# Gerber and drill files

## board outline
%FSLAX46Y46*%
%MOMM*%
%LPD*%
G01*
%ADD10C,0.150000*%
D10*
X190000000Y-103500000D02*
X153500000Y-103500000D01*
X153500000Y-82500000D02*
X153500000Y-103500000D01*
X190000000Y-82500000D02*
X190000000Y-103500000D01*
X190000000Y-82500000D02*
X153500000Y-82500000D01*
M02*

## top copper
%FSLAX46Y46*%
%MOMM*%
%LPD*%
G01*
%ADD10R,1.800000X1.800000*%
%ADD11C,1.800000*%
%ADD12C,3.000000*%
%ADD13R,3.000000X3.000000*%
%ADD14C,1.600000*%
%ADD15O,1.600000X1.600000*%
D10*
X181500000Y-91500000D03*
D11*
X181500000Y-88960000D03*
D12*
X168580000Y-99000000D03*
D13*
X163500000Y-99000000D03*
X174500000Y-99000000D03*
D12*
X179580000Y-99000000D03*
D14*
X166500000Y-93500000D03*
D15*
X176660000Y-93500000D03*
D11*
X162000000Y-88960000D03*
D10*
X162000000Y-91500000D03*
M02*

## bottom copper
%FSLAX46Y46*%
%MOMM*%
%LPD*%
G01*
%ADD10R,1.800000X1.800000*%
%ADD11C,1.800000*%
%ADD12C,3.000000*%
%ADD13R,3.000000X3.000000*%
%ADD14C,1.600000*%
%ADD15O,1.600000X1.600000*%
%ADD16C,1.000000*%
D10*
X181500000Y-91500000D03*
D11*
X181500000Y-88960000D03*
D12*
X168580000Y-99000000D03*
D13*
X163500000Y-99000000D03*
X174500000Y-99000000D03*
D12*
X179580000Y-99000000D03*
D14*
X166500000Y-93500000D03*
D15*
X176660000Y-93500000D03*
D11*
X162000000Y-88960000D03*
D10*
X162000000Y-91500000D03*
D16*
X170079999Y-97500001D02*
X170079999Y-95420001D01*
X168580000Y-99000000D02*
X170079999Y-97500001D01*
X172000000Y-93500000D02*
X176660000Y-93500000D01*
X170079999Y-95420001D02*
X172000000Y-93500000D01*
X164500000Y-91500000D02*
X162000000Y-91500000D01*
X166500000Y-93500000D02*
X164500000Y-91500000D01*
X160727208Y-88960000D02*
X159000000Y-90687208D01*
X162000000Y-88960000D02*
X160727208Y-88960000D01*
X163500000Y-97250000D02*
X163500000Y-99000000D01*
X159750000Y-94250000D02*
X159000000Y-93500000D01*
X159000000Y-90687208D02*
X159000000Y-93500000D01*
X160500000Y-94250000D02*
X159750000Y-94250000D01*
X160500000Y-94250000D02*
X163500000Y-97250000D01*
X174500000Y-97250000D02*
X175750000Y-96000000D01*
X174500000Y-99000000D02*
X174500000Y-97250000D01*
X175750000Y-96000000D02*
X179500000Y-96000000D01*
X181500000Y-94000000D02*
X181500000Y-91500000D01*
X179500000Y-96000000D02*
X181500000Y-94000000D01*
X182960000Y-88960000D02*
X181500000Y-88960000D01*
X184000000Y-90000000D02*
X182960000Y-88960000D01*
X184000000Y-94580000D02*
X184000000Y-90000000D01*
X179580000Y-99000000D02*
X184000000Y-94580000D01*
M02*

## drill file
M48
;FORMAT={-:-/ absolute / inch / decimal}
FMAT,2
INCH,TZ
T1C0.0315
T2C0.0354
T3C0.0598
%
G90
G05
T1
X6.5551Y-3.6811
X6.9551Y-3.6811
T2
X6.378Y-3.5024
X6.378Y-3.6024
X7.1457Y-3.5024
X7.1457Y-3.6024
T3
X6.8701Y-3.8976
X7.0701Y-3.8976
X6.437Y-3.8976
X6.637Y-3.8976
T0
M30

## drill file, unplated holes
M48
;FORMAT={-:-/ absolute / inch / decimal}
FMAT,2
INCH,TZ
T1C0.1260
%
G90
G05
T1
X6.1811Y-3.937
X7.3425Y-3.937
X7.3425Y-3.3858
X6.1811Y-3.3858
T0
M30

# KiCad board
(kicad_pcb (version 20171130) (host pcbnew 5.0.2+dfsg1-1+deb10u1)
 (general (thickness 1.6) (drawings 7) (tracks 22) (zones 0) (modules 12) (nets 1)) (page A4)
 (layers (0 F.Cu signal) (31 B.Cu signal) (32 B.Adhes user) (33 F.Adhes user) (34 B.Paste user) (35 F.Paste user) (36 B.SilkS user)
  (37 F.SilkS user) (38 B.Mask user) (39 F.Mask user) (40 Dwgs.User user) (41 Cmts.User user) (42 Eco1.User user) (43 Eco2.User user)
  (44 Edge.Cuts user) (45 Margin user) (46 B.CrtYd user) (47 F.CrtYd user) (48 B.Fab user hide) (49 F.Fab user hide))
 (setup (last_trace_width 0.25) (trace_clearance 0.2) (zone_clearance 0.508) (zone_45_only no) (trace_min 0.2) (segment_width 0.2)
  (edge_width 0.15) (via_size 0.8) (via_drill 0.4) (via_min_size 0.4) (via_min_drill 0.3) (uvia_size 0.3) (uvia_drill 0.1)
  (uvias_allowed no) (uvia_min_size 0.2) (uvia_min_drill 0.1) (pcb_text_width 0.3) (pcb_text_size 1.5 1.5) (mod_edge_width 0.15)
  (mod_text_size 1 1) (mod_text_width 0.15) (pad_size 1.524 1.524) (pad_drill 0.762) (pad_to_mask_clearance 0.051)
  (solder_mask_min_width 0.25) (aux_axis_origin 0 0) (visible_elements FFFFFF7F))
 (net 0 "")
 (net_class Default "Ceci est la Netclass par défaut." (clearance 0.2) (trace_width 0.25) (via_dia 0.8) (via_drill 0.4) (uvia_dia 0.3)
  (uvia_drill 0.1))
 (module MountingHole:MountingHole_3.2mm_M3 (layer F.Cu) (at 157 100)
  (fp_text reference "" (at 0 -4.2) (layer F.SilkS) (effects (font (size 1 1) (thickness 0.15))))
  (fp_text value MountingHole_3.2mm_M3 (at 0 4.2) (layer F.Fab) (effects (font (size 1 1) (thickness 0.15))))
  (pad 1 np_thru_hole circle (at 0 0) (size 3.2 3.2) (drill 3.2) (layers *.Cu *.Mask)))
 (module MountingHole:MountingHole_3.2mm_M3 (layer F.Cu) (at 186.5 100)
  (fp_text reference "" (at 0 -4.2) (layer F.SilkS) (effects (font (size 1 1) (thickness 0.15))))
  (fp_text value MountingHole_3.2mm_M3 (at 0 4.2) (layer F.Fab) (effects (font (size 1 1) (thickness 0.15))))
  (pad 1 np_thru_hole circle (at 0 0) (size 3.2 3.2) (drill 3.2) (layers *.Cu *.Mask)))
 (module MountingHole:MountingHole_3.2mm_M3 (layer F.Cu) (at 186.5 86)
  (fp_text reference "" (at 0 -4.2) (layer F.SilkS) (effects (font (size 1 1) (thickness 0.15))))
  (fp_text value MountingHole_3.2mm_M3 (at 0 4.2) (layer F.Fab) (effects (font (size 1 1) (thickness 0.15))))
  (pad 1 np_thru_hole circle (at 0 0) (size 3.2 3.2) (drill 3.2) (layers *.Cu *.Mask)))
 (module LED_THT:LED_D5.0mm (layer F.Cu) (at 181.5 91.5 90)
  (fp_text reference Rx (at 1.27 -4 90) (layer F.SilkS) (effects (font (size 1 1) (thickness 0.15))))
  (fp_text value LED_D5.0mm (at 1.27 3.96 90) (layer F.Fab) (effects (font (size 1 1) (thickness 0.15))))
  (pad 1 thru_hole rect (at 0 0 90) (size 1.8 1.8) (drill 0.9) (layers *.Cu *.Mask))
  (pad 2 thru_hole circle (at 2.54 0 90) (size 1.8 1.8) (drill 0.9) (layers *.Cu *.Mask)))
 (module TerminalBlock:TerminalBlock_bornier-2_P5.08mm (layer F.Cu) (at 163.5 99)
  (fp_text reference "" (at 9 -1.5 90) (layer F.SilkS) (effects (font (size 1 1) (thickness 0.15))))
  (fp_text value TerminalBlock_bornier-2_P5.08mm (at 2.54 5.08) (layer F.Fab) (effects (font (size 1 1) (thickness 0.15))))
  (pad 2 thru_hole circle (at 5.08 0) (size 3 3) (drill 1.52) (layers *.Cu *.Mask))
  (pad 1 thru_hole rect (at 0 0) (size 3 3) (drill 1.52) (layers *.Cu *.Mask)))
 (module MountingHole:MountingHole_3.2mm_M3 (layer F.Cu) (at 157 86)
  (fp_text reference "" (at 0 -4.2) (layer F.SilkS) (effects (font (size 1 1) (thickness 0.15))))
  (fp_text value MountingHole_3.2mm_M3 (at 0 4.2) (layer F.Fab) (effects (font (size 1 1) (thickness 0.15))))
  (pad 1 np_thru_hole circle (at 0 0) (size 3.2 3.2) (drill 3.2) (layers *.Cu *.Mask)))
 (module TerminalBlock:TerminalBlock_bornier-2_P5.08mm (layer F.Cu) (at 174.5 99)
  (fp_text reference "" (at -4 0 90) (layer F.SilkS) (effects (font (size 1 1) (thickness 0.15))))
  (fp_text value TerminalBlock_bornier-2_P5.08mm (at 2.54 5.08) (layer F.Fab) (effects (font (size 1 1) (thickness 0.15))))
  (pad 1 thru_hole rect (at 0 0) (size 3 3) (drill 1.52) (layers *.Cu *.Mask))
  (pad 2 thru_hole circle (at 5.08 0) (size 3 3) (drill 1.52) (layers *.Cu *.Mask)))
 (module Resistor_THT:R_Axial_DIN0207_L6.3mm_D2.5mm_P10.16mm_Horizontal (layer F.Cu) (at 166.5 93.5)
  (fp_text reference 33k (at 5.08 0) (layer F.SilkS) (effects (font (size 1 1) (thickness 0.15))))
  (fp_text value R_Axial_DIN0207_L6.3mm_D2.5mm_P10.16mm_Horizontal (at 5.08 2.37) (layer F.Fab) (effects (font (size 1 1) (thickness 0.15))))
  (pad 1 thru_hole circle (at 0 0) (size 1.6 1.6) (drill 0.8) (layers *.Cu *.Mask))
  (pad 2 thru_hole oval (at 10.16 0) (size 1.6 1.6) (drill 0.8) (layers *.Cu *.Mask)))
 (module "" (layer F.Cu) (at 72 144.5)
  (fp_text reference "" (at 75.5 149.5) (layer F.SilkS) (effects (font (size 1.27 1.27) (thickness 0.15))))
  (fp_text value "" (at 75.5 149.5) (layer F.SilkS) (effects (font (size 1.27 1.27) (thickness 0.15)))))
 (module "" (layer F.Cu) (at 45.5 145)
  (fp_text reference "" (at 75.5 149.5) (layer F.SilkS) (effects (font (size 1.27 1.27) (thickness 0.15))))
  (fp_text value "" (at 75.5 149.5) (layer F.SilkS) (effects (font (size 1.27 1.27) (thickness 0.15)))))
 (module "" (layer F.Cu) (at 80 110.5)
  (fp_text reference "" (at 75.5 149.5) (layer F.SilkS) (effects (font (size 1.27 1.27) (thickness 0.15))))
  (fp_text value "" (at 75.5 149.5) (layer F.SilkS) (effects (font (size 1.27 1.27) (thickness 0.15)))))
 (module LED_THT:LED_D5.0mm (layer F.Cu) (at 162 91.5 90)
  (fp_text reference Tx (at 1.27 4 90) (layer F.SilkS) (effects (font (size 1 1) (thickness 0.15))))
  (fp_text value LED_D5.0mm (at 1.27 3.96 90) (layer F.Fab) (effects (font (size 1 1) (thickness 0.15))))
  (pad 2 thru_hole circle (at 2.54 0 90) (size 1.8 1.8) (drill 0.9) (layers *.Cu *.Mask))
  (pad 1 thru_hole rect (at 0 0 90) (size 1.8 1.8) (drill 0.9) (layers *.Cu *.Mask)))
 (gr_line (start 190 103.5) (end 153.5 103.5) (layer Edge.Cuts) (width 0.15))
 (gr_line (start 153.5 82.5) (end 153.5 103.5) (layer Edge.Cuts) (width 0.15))
 (gr_line (start 190 82.5) (end 190 103.5) (layer Edge.Cuts) (width 0.15))
 (gr_line (start 190 82.5) (end 153.5 82.5) (layer Edge.Cuts) (width 0.15))
 (segment (start 170.079999 97.500001) (end 170.079999 95.420001) (width 1) (layer B.Cu) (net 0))
 (segment (start 168.58 99) (end 170.079999 97.500001) (width 1) (layer B.Cu) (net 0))
 (segment (start 172 93.5) (end 176.66 93.5) (width 1) (layer B.Cu) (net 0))
 (segment (start 170.079999 95.420001) (end 172 93.5) (width 1) (layer B.Cu) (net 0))
 (segment (start 164.5 91.5) (end 162 91.5) (width 1) (layer B.Cu) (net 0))
 (segment (start 166.5 93.5) (end 164.5 91.5) (width 1) (layer B.Cu) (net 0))
 (segment (start 160.727208 88.96) (end 159 90.687208) (width 1) (layer B.Cu) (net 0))
 (segment (start 162 88.96) (end 160.727208 88.96) (width 1) (layer B.Cu) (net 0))
 (segment (start 163.5 97.25) (end 163.5 99) (width 1) (layer B.Cu) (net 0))
 (segment (start 159.75 94.25) (end 159 93.5) (width 1) (layer B.Cu) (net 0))
 (segment (start 159 90.687208) (end 159 93.5) (width 1) (layer B.Cu) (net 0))
 (segment (start 160.5 94.25) (end 159.75 94.25) (width 1) (layer B.Cu) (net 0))
 (segment (start 160.5 94.25) (end 163.5 97.25) (width 1) (layer B.Cu) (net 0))
 (segment (start 174.5 97.25) (end 175.75 96) (width 1) (layer B.Cu) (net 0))
 (segment (start 174.5 99) (end 174.5 97.25) (width 1) (layer B.Cu) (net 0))
 (segment (start 175.75 96) (end 179.5 96) (width 1) (layer B.Cu) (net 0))
 (segment (start 181.5 94) (end 181.5 91.5) (width 1) (layer B.Cu) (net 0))
 (segment (start 179.5 96) (end 181.5 94) (width 1) (layer B.Cu) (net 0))
 (segment (start 182.96 88.96) (end 181.5 88.96) (width 1) (layer B.Cu) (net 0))
 (segment (start 184 90) (end 182.96 88.96) (width 1) (layer B.Cu) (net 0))
 (segment (start 184 94.58) (end 184 90) (width 1) (layer B.Cu) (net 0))
 (segment (start 179.58 99) (end 184 94.58) (width 1) (layer B.Cu) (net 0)))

